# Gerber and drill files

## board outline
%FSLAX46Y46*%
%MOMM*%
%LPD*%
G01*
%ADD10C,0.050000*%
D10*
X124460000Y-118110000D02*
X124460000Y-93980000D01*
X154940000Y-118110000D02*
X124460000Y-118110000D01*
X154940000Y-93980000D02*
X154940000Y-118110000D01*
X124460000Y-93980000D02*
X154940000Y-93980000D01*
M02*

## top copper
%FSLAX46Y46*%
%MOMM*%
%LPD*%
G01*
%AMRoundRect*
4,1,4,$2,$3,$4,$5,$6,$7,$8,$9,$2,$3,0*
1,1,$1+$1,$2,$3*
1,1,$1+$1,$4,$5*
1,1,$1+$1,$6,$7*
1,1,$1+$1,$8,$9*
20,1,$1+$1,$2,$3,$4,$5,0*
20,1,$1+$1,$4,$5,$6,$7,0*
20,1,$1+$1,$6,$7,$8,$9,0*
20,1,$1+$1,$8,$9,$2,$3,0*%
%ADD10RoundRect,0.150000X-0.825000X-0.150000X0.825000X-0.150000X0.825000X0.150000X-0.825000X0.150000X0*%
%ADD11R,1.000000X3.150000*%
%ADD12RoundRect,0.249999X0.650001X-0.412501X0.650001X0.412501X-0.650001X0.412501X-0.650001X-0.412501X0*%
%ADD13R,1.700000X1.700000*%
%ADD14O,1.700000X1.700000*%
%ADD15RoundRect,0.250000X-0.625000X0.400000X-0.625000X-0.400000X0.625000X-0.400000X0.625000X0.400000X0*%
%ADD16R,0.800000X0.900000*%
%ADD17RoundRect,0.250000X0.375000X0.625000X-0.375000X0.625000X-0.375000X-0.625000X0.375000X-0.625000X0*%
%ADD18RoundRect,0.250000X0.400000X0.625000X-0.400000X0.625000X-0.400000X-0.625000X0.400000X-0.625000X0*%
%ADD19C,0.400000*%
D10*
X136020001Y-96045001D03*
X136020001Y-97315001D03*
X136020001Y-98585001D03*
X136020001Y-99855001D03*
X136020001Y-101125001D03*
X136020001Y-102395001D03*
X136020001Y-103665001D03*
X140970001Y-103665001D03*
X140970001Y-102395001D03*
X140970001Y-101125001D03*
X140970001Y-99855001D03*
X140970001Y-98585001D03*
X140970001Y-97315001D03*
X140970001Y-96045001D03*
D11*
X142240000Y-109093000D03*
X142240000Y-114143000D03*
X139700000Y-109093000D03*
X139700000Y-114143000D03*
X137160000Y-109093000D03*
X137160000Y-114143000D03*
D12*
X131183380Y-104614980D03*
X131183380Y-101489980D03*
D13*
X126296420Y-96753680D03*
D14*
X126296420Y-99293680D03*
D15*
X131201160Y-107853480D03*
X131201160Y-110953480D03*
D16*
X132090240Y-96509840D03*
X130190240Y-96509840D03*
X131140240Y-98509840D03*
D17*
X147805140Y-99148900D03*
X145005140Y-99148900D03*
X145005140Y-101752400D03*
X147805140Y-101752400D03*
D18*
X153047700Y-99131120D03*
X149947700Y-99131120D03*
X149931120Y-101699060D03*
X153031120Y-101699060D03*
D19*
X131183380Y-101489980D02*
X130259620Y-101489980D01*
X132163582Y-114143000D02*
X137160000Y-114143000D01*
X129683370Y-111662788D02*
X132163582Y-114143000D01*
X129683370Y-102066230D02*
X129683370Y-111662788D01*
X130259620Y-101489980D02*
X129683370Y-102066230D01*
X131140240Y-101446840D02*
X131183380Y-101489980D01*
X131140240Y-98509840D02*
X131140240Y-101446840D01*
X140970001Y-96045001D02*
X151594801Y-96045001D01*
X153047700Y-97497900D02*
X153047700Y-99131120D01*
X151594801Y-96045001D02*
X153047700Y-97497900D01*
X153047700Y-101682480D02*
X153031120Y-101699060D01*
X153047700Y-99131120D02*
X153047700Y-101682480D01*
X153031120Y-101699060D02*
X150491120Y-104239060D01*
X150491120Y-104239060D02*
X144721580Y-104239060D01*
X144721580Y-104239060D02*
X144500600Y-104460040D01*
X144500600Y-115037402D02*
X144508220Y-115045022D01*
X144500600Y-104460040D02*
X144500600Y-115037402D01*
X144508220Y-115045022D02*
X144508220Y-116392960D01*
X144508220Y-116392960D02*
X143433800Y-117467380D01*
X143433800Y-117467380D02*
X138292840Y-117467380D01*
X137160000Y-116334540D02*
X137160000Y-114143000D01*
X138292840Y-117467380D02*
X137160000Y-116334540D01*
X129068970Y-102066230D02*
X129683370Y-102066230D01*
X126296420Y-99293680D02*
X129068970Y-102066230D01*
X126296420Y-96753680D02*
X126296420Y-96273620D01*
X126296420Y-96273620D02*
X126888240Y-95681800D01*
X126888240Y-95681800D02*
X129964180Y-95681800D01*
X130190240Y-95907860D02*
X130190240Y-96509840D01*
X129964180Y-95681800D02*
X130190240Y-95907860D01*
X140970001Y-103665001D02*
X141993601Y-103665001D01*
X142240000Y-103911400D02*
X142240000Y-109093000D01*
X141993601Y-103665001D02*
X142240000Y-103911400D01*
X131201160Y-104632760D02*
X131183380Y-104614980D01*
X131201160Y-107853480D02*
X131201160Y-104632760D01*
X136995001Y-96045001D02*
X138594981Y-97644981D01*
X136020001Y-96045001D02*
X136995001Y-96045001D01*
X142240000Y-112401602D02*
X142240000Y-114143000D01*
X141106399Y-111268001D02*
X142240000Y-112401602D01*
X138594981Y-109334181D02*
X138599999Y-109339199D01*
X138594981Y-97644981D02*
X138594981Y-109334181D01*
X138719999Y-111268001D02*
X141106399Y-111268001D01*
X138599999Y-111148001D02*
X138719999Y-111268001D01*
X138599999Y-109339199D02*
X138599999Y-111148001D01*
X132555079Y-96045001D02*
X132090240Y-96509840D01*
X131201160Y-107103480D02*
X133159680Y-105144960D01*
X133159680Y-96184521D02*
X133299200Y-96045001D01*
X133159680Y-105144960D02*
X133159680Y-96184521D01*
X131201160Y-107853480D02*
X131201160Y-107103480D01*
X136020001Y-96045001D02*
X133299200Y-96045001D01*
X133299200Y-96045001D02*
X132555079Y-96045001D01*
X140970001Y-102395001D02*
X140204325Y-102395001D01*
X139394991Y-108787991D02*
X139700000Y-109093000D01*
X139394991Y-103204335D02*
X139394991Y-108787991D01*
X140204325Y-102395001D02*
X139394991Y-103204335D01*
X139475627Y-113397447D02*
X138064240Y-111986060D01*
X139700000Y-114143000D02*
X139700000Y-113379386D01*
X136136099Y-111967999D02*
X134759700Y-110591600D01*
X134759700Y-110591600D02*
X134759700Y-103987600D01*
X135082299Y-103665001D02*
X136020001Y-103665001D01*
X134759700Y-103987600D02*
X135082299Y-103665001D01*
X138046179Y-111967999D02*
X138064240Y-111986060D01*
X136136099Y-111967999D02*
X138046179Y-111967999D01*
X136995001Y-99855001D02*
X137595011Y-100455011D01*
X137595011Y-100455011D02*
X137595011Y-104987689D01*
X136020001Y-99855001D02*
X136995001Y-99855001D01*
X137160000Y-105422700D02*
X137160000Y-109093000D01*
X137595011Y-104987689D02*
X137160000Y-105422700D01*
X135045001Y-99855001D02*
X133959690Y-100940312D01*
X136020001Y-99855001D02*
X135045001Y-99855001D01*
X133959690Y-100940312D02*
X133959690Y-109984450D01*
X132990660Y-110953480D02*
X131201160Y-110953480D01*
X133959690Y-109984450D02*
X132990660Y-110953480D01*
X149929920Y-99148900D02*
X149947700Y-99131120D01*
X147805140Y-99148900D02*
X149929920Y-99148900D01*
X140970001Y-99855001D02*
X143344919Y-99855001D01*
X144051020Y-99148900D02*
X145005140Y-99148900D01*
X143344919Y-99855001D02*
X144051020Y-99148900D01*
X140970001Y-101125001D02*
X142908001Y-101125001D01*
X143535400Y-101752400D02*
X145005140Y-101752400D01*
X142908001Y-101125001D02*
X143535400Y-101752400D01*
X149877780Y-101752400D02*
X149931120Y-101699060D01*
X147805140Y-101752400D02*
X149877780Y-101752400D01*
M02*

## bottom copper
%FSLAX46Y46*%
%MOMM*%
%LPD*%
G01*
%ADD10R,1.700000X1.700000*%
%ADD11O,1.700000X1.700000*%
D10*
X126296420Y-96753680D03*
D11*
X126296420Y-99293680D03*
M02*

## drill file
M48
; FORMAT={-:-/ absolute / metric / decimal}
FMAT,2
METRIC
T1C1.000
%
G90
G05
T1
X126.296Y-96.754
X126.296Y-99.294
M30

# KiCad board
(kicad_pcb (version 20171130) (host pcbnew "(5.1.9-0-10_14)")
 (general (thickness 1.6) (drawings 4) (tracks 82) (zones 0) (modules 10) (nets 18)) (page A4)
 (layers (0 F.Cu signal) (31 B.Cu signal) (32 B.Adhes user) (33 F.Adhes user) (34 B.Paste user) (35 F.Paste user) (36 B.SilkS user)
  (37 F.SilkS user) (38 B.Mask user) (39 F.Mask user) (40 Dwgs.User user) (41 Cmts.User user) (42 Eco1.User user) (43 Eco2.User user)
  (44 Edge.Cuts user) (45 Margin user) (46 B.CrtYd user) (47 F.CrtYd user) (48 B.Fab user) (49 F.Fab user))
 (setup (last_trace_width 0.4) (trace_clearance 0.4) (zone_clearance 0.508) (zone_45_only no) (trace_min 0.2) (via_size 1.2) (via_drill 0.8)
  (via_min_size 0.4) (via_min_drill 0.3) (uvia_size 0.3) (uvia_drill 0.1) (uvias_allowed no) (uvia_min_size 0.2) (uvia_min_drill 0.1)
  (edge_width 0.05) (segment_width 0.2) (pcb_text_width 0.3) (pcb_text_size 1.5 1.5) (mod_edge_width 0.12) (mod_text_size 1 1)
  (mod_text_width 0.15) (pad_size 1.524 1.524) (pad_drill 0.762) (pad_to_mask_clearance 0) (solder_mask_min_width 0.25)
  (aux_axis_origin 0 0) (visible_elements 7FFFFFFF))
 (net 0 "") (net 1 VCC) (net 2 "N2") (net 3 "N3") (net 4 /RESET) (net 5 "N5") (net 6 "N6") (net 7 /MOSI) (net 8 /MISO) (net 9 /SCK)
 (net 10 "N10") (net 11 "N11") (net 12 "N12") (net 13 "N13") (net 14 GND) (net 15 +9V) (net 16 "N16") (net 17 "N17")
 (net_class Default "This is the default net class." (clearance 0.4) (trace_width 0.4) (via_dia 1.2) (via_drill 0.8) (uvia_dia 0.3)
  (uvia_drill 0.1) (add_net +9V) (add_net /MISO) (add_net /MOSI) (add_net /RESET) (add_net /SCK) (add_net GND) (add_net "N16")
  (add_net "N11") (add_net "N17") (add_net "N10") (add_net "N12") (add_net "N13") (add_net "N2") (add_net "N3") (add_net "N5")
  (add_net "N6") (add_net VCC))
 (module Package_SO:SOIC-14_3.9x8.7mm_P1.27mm (layer F.Cu) (at 138.495001 99.855001)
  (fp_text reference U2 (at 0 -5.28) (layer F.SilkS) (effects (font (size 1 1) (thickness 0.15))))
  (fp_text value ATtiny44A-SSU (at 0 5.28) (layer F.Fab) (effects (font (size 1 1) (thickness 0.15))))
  (pad 1 smd roundrect (at -2.475 -3.81) (size 1.95 0.6) (layers F.Cu F.Paste F.Mask) (roundrect_rratio 0.25) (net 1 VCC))
  (pad 2 smd roundrect (at -2.475 -2.54) (size 1.95 0.6) (layers F.Cu F.Paste F.Mask) (roundrect_rratio 0.25) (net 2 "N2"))
  (pad 3 smd roundrect (at -2.475 -1.27) (size 1.95 0.6) (layers F.Cu F.Paste F.Mask) (roundrect_rratio 0.25) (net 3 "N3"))
  (pad 4 smd roundrect (at -2.475 0) (size 1.95 0.6) (layers F.Cu F.Paste F.Mask) (roundrect_rratio 0.25) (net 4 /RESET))
  (pad 5 smd roundrect (at -2.475 1.27) (size 1.95 0.6) (layers F.Cu F.Paste F.Mask) (roundrect_rratio 0.25) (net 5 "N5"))
  (pad 6 smd roundrect (at -2.475 2.54) (size 1.95 0.6) (layers F.Cu F.Paste F.Mask) (roundrect_rratio 0.25) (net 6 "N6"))
  (pad 7 smd roundrect (at -2.475 3.81) (size 1.95 0.6) (layers F.Cu F.Paste F.Mask) (roundrect_rratio 0.25) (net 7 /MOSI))
  (pad 8 smd roundrect (at 2.475 3.81) (size 1.95 0.6) (layers F.Cu F.Paste F.Mask) (roundrect_rratio 0.25) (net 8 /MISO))
  (pad 9 smd roundrect (at 2.475 2.54) (size 1.95 0.6) (layers F.Cu F.Paste F.Mask) (roundrect_rratio 0.25) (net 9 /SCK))
  (pad 10 smd roundrect (at 2.475 1.27) (size 1.95 0.6) (layers F.Cu F.Paste F.Mask) (roundrect_rratio 0.25) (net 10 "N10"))
  (pad 11 smd roundrect (at 2.475 0) (size 1.95 0.6) (layers F.Cu F.Paste F.Mask) (roundrect_rratio 0.25) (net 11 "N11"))
  (pad 12 smd roundrect (at 2.475 -1.27) (size 1.95 0.6) (layers F.Cu F.Paste F.Mask) (roundrect_rratio 0.25) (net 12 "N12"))
  (pad 13 smd roundrect (at 2.475 -2.54) (size 1.95 0.6) (layers F.Cu F.Paste F.Mask) (roundrect_rratio 0.25) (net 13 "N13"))
  (pad 14 smd roundrect (at 2.475 -3.81) (size 1.95 0.6) (layers F.Cu F.Paste F.Mask) (roundrect_rratio 0.25) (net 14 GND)))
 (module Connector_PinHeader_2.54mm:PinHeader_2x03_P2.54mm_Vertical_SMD (layer F.Cu) (at 139.7 111.618 270)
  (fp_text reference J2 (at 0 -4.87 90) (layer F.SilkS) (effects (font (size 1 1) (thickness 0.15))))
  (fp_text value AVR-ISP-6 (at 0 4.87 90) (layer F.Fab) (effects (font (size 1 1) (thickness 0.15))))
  (pad 1 smd rect (at -2.525 -2.54 270) (size 3.15 1) (layers F.Cu F.Paste F.Mask) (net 8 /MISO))
  (pad 2 smd rect (at 2.525 -2.54 270) (size 3.15 1) (layers F.Cu F.Paste F.Mask) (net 1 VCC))
  (pad 3 smd rect (at -2.525 0 270) (size 3.15 1) (layers F.Cu F.Paste F.Mask) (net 9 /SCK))
  (pad 4 smd rect (at 2.525 0 270) (size 3.15 1) (layers F.Cu F.Paste F.Mask) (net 7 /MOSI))
  (pad 5 smd rect (at -2.525 2.54 270) (size 3.15 1) (layers F.Cu F.Paste F.Mask) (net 4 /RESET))
  (pad 6 smd rect (at 2.525 2.54 270) (size 3.15 1) (layers F.Cu F.Paste F.Mask) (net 14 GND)))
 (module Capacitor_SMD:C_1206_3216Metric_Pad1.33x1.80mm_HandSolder (layer F.Cu) (at 131.18338 103.05248 90)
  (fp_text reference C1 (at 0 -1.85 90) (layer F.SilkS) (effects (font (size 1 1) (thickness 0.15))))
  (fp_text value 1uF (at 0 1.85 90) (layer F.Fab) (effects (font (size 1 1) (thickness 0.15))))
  (pad 1 smd roundrect (at -1.5625 0 90) (size 1.325 1.8) (layers F.Cu F.Paste F.Mask) (roundrect_rratio 0.1886784905660377) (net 1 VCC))
  (pad 2 smd roundrect (at 1.5625 0 90) (size 1.325 1.8) (layers F.Cu F.Paste F.Mask) (roundrect_rratio 0.1886784905660377) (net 14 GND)))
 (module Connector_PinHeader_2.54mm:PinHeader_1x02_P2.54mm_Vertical (layer F.Cu) (at 126.29642 96.75368)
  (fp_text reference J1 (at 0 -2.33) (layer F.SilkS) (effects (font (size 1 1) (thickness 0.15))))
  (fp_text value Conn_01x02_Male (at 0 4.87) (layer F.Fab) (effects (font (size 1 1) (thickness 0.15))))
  (pad 1 thru_hole rect (at 0 0) (size 1.7 1.7) (drill 1) (layers *.Cu *.Mask) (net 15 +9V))
  (pad 2 thru_hole oval (at 0 2.54) (size 1.7 1.7) (drill 1) (layers *.Cu *.Mask) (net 14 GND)))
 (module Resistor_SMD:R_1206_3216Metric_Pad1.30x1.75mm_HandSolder (layer F.Cu) (at 131.20116 109.40348 270)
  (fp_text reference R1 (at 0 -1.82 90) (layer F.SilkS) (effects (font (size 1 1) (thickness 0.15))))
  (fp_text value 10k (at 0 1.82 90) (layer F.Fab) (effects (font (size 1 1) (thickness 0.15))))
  (pad 1 smd roundrect (at -1.55 0 270) (size 1.3 1.75) (layers F.Cu F.Paste F.Mask) (roundrect_rratio 0.1923076923076923) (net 1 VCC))
  (pad 2 smd roundrect (at 1.55 0 270) (size 1.3 1.75) (layers F.Cu F.Paste F.Mask) (roundrect_rratio 0.1923076923076923) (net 4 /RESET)))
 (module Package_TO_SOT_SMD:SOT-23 (layer F.Cu) (at 131.14024 97.50984 270)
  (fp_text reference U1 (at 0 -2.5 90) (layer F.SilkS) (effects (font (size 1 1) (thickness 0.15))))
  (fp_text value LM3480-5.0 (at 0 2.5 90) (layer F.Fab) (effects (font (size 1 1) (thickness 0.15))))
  (pad 1 smd rect (at -1 -0.95 270) (size 0.9 0.8) (layers F.Cu F.Paste F.Mask) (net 1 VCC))
  (pad 2 smd rect (at -1 0.95 270) (size 0.9 0.8) (layers F.Cu F.Paste F.Mask) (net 15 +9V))
  (pad 3 smd rect (at 1 0 270) (size 0.9 0.8) (layers F.Cu F.Paste F.Mask) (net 14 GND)))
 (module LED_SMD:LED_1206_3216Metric (layer F.Cu) (at 146.40514 99.1489 180)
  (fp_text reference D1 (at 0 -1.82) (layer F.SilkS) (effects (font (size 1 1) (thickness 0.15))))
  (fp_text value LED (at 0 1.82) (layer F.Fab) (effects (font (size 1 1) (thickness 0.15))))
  (pad 1 smd roundrect (at -1.4 0 180) (size 1.25 1.75) (layers F.Cu F.Paste F.Mask) (roundrect_rratio 0.2) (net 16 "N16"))
  (pad 2 smd roundrect (at 1.4 0 180) (size 1.25 1.75) (layers F.Cu F.Paste F.Mask) (roundrect_rratio 0.2) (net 11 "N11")))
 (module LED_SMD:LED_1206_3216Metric (layer F.Cu) (at 146.40514 101.7524 180)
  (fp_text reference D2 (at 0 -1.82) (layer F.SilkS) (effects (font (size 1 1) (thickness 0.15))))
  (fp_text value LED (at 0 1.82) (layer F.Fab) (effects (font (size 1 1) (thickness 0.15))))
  (pad 2 smd roundrect (at 1.4 0 180) (size 1.25 1.75) (layers F.Cu F.Paste F.Mask) (roundrect_rratio 0.2) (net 10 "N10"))
  (pad 1 smd roundrect (at -1.4 0 180) (size 1.25 1.75) (layers F.Cu F.Paste F.Mask) (roundrect_rratio 0.2) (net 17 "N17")))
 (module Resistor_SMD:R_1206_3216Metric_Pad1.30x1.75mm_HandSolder (layer F.Cu) (at 151.4977 99.13112 180)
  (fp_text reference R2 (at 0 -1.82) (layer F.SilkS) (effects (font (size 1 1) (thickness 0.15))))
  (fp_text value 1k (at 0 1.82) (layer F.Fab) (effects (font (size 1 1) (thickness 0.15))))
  (pad 1 smd roundrect (at -1.55 0 180) (size 1.3 1.75) (layers F.Cu F.Paste F.Mask) (roundrect_rratio 0.1923076923076923) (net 14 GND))
  (pad 2 smd roundrect (at 1.55 0 180) (size 1.3 1.75) (layers F.Cu F.Paste F.Mask) (roundrect_rratio 0.1923076923076923) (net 16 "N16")))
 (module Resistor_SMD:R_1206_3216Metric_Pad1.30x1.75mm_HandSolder (layer F.Cu) (at 151.48112 101.69906 180)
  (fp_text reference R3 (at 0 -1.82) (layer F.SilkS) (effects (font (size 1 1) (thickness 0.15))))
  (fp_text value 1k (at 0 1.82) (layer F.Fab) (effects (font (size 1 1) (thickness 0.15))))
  (pad 2 smd roundrect (at 1.55 0 180) (size 1.3 1.75) (layers F.Cu F.Paste F.Mask) (roundrect_rratio 0.1923076923076923) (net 17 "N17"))
  (pad 1 smd roundrect (at -1.55 0 180) (size 1.3 1.75) (layers F.Cu F.Paste F.Mask) (roundrect_rratio 0.1923076923076923) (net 14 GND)))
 (gr_line (start 124.46 118.11) (end 124.46 93.98) (layer Edge.Cuts) (width 0.05))
 (gr_line (start 154.94 118.11) (end 124.46 118.11) (layer Edge.Cuts) (width 0.05))
 (gr_line (start 154.94 93.98) (end 154.94 118.11) (layer Edge.Cuts) (width 0.05))
 (gr_line (start 124.46 93.98) (end 154.94 93.98) (layer Edge.Cuts) (width 0.05))
 (segment (start 131.18338 101.48998) (end 130.25962 101.48998) (width 0.4) (layer F.Cu) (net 14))
 (segment (start 132.163582 114.143) (end 137.16 114.143) (width 0.4) (layer F.Cu) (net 14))
 (segment (start 129.68337 111.662788) (end 132.163582 114.143) (width 0.4) (layer F.Cu) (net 14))
 (segment (start 129.68337 102.06623) (end 129.68337 111.662788) (width 0.4) (layer F.Cu) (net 14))
 (segment (start 130.25962 101.48998) (end 129.68337 102.06623) (width 0.4) (layer F.Cu) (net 14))
 (segment (start 131.14024 101.44684) (end 131.18338 101.48998) (width 0.4) (layer F.Cu) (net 14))
 (segment (start 131.14024 98.50984) (end 131.14024 101.44684) (width 0.4) (layer F.Cu) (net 14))
 (segment (start 140.970001 96.045001) (end 151.594801 96.045001) (width 0.4) (layer F.Cu) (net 14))
 (segment (start 153.0477 97.4979) (end 153.0477 99.13112) (width 0.4) (layer F.Cu) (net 14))
 (segment (start 151.594801 96.045001) (end 153.0477 97.4979) (width 0.4) (layer F.Cu) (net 14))
 (segment (start 153.0477 101.68248) (end 153.03112 101.69906) (width 0.4) (layer F.Cu) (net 14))
 (segment (start 153.0477 99.13112) (end 153.0477 101.68248) (width 0.4) (layer F.Cu) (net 14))
 (segment (start 153.03112 101.69906) (end 150.49112 104.23906) (width 0.4) (layer F.Cu) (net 14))
 (segment (start 150.49112 104.23906) (end 144.72158 104.23906) (width 0.4) (layer F.Cu) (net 14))
 (segment (start 144.72158 104.23906) (end 144.5006 104.46004) (width 0.4) (layer F.Cu) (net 14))
 (segment (start 144.5006 115.037402) (end 144.50822 115.045022) (width 0.4) (layer F.Cu) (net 14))
 (segment (start 144.5006 104.46004) (end 144.5006 115.037402) (width 0.4) (layer F.Cu) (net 14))
 (segment (start 144.50822 115.045022) (end 144.50822 116.39296) (width 0.4) (layer F.Cu) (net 14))
 (segment (start 144.50822 116.39296) (end 143.4338 117.46738) (width 0.4) (layer F.Cu) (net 14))
 (segment (start 143.4338 117.46738) (end 138.29284 117.46738) (width 0.4) (layer F.Cu) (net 14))
 (segment (start 137.16 116.33454) (end 137.16 114.143) (width 0.4) (layer F.Cu) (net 14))
 (segment (start 138.29284 117.46738) (end 137.16 116.33454) (width 0.4) (layer F.Cu) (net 14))
 (segment (start 129.06897 102.06623) (end 129.68337 102.06623) (width 0.4) (layer F.Cu) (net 14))
 (segment (start 126.29642 99.29368) (end 129.06897 102.06623) (width 0.4) (layer F.Cu) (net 14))
 (segment (start 126.29642 96.75368) (end 126.29642 96.27362) (width 0.4) (layer F.Cu) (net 15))
 (segment (start 126.29642 96.27362) (end 126.88824 95.6818) (width 0.4) (layer F.Cu) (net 15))
 (segment (start 126.88824 95.6818) (end 129.96418 95.6818) (width 0.4) (layer F.Cu) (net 15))
 (segment (start 130.19024 95.90786) (end 130.19024 96.50984) (width 0.4) (layer F.Cu) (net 15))
 (segment (start 129.96418 95.6818) (end 130.19024 95.90786) (width 0.4) (layer F.Cu) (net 15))
 (segment (start 140.970001 103.665001) (end 141.993601 103.665001) (width 0.4) (layer F.Cu) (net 8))
 (segment (start 142.24 103.9114) (end 142.24 109.093) (width 0.4) (layer F.Cu) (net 8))
 (segment (start 141.993601 103.665001) (end 142.24 103.9114) (width 0.4) (layer F.Cu) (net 8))
 (segment (start 131.20116 104.63276) (end 131.18338 104.61498) (width 0.4) (layer F.Cu) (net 1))
 (segment (start 131.20116 107.85348) (end 131.20116 104.63276) (width 0.4) (layer F.Cu) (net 1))
 (segment (start 136.995001 96.045001) (end 138.594981 97.644981) (width 0.4) (layer F.Cu) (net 1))
 (segment (start 136.020001 96.045001) (end 136.995001 96.045001) (width 0.4) (layer F.Cu) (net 1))
 (segment (start 142.24 112.401602) (end 142.24 114.143) (width 0.4) (layer F.Cu) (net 1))
 (segment (start 141.106399 111.268001) (end 142.24 112.401602) (width 0.4) (layer F.Cu) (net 1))
 (segment (start 138.594981 109.334181) (end 138.599999 109.339199) (width 0.4) (layer F.Cu) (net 1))
 (segment (start 138.594981 97.644981) (end 138.594981 109.334181) (width 0.4) (layer F.Cu) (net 1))
 (segment (start 138.719999 111.268001) (end 141.106399 111.268001) (width 0.4) (layer F.Cu) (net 1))
 (segment (start 138.599999 111.148001) (end 138.719999 111.268001) (width 0.4) (layer F.Cu) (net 1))
 (segment (start 138.599999 109.339199) (end 138.599999 111.148001) (width 0.4) (layer F.Cu) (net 1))
 (segment (start 132.555079 96.045001) (end 132.09024 96.50984) (width 0.4) (layer F.Cu) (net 1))
 (segment (start 131.20116 107.10348) (end 133.15968 105.14496) (width 0.4) (layer F.Cu) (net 1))
 (segment (start 133.15968 96.184521) (end 133.2992 96.045001) (width 0.4) (layer F.Cu) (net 1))
 (segment (start 133.15968 105.14496) (end 133.15968 96.184521) (width 0.4) (layer F.Cu) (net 1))
 (segment (start 131.20116 107.85348) (end 131.20116 107.10348) (width 0.4) (layer F.Cu) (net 1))
 (segment (start 136.020001 96.045001) (end 133.2992 96.045001) (width 0.4) (layer F.Cu) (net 1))
 (segment (start 133.2992 96.045001) (end 132.555079 96.045001) (width 0.4) (layer F.Cu) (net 1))
 (segment (start 140.970001 102.395001) (end 140.204325 102.395001) (width 0.4) (layer F.Cu) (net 9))
 (segment (start 139.394991 108.787991) (end 139.7 109.093) (width 0.4) (layer F.Cu) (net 9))
 (segment (start 139.394991 103.204335) (end 139.394991 108.787991) (width 0.4) (layer F.Cu) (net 9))
 (segment (start 140.204325 102.395001) (end 139.394991 103.204335) (width 0.4) (layer F.Cu) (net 9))
 (segment (start 139.475627 113.397447) (end 138.06424 111.98606) (width 0.4) (layer F.Cu) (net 7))
 (segment (start 139.7 114.143) (end 139.7 113.379386) (width 0.4) (layer F.Cu) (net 7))
 (segment (start 136.136099 111.967999) (end 134.7597 110.5916) (width 0.4) (layer F.Cu) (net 7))
 (segment (start 134.7597 110.5916) (end 134.7597 103.9876) (width 0.4) (layer F.Cu) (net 7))
 (segment (start 135.082299 103.665001) (end 136.020001 103.665001) (width 0.4) (layer F.Cu) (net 7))
 (segment (start 134.7597 103.9876) (end 135.082299 103.665001) (width 0.4) (layer F.Cu) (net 7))
 (segment (start 138.046179 111.967999) (end 138.06424 111.98606) (width 0.4) (layer F.Cu) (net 7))
 (segment (start 136.136099 111.967999) (end 138.046179 111.967999) (width 0.4) (layer F.Cu) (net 7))
 (segment (start 136.995001 99.855001) (end 137.595011 100.455011) (width 0.4) (layer F.Cu) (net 4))
 (segment (start 137.595011 100.455011) (end 137.595011 104.987689) (width 0.4) (layer F.Cu) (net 4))
 (segment (start 136.020001 99.855001) (end 136.995001 99.855001) (width 0.4) (layer F.Cu) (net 4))
 (segment (start 137.16 105.4227) (end 137.16 109.093) (width 0.4) (layer F.Cu) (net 4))
 (segment (start 137.595011 104.987689) (end 137.16 105.4227) (width 0.4) (layer F.Cu) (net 4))
 (segment (start 135.045001 99.855001) (end 133.95969 100.940312) (width 0.4) (layer F.Cu) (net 4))
 (segment (start 136.020001 99.855001) (end 135.045001 99.855001) (width 0.4) (layer F.Cu) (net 4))
 (segment (start 133.95969 100.940312) (end 133.95969 109.98445) (width 0.4) (layer F.Cu) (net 4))
 (segment (start 132.99066 110.95348) (end 131.20116 110.95348) (width 0.4) (layer F.Cu) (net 4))
 (segment (start 133.95969 109.98445) (end 132.99066 110.95348) (width 0.4) (layer F.Cu) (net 4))
 (segment (start 149.92992 99.1489) (end 149.9477 99.13112) (width 0.4) (layer F.Cu) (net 16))
 (segment (start 147.80514 99.1489) (end 149.92992 99.1489) (width 0.4) (layer F.Cu) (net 16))
 (segment (start 140.970001 99.855001) (end 143.344919 99.855001) (width 0.4) (layer F.Cu) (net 11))
 (segment (start 144.05102 99.1489) (end 145.00514 99.1489) (width 0.4) (layer F.Cu) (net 11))
 (segment (start 143.344919 99.855001) (end 144.05102 99.1489) (width 0.4) (layer F.Cu) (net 11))
 (segment (start 140.970001 101.125001) (end 142.908001 101.125001) (width 0.4) (layer F.Cu) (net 10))
 (segment (start 143.5354 101.7524) (end 145.00514 101.7524) (width 0.4) (layer F.Cu) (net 10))
 (segment (start 142.908001 101.125001) (end 143.5354 101.7524) (width 0.4) (layer F.Cu) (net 10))
 (segment (start 149.87778 101.7524) (end 149.93112 101.69906) (width 0.4) (layer F.Cu) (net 17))
 (segment (start 147.80514 101.7524) (end 149.87778 101.7524) (width 0.4) (layer F.Cu) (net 17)))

